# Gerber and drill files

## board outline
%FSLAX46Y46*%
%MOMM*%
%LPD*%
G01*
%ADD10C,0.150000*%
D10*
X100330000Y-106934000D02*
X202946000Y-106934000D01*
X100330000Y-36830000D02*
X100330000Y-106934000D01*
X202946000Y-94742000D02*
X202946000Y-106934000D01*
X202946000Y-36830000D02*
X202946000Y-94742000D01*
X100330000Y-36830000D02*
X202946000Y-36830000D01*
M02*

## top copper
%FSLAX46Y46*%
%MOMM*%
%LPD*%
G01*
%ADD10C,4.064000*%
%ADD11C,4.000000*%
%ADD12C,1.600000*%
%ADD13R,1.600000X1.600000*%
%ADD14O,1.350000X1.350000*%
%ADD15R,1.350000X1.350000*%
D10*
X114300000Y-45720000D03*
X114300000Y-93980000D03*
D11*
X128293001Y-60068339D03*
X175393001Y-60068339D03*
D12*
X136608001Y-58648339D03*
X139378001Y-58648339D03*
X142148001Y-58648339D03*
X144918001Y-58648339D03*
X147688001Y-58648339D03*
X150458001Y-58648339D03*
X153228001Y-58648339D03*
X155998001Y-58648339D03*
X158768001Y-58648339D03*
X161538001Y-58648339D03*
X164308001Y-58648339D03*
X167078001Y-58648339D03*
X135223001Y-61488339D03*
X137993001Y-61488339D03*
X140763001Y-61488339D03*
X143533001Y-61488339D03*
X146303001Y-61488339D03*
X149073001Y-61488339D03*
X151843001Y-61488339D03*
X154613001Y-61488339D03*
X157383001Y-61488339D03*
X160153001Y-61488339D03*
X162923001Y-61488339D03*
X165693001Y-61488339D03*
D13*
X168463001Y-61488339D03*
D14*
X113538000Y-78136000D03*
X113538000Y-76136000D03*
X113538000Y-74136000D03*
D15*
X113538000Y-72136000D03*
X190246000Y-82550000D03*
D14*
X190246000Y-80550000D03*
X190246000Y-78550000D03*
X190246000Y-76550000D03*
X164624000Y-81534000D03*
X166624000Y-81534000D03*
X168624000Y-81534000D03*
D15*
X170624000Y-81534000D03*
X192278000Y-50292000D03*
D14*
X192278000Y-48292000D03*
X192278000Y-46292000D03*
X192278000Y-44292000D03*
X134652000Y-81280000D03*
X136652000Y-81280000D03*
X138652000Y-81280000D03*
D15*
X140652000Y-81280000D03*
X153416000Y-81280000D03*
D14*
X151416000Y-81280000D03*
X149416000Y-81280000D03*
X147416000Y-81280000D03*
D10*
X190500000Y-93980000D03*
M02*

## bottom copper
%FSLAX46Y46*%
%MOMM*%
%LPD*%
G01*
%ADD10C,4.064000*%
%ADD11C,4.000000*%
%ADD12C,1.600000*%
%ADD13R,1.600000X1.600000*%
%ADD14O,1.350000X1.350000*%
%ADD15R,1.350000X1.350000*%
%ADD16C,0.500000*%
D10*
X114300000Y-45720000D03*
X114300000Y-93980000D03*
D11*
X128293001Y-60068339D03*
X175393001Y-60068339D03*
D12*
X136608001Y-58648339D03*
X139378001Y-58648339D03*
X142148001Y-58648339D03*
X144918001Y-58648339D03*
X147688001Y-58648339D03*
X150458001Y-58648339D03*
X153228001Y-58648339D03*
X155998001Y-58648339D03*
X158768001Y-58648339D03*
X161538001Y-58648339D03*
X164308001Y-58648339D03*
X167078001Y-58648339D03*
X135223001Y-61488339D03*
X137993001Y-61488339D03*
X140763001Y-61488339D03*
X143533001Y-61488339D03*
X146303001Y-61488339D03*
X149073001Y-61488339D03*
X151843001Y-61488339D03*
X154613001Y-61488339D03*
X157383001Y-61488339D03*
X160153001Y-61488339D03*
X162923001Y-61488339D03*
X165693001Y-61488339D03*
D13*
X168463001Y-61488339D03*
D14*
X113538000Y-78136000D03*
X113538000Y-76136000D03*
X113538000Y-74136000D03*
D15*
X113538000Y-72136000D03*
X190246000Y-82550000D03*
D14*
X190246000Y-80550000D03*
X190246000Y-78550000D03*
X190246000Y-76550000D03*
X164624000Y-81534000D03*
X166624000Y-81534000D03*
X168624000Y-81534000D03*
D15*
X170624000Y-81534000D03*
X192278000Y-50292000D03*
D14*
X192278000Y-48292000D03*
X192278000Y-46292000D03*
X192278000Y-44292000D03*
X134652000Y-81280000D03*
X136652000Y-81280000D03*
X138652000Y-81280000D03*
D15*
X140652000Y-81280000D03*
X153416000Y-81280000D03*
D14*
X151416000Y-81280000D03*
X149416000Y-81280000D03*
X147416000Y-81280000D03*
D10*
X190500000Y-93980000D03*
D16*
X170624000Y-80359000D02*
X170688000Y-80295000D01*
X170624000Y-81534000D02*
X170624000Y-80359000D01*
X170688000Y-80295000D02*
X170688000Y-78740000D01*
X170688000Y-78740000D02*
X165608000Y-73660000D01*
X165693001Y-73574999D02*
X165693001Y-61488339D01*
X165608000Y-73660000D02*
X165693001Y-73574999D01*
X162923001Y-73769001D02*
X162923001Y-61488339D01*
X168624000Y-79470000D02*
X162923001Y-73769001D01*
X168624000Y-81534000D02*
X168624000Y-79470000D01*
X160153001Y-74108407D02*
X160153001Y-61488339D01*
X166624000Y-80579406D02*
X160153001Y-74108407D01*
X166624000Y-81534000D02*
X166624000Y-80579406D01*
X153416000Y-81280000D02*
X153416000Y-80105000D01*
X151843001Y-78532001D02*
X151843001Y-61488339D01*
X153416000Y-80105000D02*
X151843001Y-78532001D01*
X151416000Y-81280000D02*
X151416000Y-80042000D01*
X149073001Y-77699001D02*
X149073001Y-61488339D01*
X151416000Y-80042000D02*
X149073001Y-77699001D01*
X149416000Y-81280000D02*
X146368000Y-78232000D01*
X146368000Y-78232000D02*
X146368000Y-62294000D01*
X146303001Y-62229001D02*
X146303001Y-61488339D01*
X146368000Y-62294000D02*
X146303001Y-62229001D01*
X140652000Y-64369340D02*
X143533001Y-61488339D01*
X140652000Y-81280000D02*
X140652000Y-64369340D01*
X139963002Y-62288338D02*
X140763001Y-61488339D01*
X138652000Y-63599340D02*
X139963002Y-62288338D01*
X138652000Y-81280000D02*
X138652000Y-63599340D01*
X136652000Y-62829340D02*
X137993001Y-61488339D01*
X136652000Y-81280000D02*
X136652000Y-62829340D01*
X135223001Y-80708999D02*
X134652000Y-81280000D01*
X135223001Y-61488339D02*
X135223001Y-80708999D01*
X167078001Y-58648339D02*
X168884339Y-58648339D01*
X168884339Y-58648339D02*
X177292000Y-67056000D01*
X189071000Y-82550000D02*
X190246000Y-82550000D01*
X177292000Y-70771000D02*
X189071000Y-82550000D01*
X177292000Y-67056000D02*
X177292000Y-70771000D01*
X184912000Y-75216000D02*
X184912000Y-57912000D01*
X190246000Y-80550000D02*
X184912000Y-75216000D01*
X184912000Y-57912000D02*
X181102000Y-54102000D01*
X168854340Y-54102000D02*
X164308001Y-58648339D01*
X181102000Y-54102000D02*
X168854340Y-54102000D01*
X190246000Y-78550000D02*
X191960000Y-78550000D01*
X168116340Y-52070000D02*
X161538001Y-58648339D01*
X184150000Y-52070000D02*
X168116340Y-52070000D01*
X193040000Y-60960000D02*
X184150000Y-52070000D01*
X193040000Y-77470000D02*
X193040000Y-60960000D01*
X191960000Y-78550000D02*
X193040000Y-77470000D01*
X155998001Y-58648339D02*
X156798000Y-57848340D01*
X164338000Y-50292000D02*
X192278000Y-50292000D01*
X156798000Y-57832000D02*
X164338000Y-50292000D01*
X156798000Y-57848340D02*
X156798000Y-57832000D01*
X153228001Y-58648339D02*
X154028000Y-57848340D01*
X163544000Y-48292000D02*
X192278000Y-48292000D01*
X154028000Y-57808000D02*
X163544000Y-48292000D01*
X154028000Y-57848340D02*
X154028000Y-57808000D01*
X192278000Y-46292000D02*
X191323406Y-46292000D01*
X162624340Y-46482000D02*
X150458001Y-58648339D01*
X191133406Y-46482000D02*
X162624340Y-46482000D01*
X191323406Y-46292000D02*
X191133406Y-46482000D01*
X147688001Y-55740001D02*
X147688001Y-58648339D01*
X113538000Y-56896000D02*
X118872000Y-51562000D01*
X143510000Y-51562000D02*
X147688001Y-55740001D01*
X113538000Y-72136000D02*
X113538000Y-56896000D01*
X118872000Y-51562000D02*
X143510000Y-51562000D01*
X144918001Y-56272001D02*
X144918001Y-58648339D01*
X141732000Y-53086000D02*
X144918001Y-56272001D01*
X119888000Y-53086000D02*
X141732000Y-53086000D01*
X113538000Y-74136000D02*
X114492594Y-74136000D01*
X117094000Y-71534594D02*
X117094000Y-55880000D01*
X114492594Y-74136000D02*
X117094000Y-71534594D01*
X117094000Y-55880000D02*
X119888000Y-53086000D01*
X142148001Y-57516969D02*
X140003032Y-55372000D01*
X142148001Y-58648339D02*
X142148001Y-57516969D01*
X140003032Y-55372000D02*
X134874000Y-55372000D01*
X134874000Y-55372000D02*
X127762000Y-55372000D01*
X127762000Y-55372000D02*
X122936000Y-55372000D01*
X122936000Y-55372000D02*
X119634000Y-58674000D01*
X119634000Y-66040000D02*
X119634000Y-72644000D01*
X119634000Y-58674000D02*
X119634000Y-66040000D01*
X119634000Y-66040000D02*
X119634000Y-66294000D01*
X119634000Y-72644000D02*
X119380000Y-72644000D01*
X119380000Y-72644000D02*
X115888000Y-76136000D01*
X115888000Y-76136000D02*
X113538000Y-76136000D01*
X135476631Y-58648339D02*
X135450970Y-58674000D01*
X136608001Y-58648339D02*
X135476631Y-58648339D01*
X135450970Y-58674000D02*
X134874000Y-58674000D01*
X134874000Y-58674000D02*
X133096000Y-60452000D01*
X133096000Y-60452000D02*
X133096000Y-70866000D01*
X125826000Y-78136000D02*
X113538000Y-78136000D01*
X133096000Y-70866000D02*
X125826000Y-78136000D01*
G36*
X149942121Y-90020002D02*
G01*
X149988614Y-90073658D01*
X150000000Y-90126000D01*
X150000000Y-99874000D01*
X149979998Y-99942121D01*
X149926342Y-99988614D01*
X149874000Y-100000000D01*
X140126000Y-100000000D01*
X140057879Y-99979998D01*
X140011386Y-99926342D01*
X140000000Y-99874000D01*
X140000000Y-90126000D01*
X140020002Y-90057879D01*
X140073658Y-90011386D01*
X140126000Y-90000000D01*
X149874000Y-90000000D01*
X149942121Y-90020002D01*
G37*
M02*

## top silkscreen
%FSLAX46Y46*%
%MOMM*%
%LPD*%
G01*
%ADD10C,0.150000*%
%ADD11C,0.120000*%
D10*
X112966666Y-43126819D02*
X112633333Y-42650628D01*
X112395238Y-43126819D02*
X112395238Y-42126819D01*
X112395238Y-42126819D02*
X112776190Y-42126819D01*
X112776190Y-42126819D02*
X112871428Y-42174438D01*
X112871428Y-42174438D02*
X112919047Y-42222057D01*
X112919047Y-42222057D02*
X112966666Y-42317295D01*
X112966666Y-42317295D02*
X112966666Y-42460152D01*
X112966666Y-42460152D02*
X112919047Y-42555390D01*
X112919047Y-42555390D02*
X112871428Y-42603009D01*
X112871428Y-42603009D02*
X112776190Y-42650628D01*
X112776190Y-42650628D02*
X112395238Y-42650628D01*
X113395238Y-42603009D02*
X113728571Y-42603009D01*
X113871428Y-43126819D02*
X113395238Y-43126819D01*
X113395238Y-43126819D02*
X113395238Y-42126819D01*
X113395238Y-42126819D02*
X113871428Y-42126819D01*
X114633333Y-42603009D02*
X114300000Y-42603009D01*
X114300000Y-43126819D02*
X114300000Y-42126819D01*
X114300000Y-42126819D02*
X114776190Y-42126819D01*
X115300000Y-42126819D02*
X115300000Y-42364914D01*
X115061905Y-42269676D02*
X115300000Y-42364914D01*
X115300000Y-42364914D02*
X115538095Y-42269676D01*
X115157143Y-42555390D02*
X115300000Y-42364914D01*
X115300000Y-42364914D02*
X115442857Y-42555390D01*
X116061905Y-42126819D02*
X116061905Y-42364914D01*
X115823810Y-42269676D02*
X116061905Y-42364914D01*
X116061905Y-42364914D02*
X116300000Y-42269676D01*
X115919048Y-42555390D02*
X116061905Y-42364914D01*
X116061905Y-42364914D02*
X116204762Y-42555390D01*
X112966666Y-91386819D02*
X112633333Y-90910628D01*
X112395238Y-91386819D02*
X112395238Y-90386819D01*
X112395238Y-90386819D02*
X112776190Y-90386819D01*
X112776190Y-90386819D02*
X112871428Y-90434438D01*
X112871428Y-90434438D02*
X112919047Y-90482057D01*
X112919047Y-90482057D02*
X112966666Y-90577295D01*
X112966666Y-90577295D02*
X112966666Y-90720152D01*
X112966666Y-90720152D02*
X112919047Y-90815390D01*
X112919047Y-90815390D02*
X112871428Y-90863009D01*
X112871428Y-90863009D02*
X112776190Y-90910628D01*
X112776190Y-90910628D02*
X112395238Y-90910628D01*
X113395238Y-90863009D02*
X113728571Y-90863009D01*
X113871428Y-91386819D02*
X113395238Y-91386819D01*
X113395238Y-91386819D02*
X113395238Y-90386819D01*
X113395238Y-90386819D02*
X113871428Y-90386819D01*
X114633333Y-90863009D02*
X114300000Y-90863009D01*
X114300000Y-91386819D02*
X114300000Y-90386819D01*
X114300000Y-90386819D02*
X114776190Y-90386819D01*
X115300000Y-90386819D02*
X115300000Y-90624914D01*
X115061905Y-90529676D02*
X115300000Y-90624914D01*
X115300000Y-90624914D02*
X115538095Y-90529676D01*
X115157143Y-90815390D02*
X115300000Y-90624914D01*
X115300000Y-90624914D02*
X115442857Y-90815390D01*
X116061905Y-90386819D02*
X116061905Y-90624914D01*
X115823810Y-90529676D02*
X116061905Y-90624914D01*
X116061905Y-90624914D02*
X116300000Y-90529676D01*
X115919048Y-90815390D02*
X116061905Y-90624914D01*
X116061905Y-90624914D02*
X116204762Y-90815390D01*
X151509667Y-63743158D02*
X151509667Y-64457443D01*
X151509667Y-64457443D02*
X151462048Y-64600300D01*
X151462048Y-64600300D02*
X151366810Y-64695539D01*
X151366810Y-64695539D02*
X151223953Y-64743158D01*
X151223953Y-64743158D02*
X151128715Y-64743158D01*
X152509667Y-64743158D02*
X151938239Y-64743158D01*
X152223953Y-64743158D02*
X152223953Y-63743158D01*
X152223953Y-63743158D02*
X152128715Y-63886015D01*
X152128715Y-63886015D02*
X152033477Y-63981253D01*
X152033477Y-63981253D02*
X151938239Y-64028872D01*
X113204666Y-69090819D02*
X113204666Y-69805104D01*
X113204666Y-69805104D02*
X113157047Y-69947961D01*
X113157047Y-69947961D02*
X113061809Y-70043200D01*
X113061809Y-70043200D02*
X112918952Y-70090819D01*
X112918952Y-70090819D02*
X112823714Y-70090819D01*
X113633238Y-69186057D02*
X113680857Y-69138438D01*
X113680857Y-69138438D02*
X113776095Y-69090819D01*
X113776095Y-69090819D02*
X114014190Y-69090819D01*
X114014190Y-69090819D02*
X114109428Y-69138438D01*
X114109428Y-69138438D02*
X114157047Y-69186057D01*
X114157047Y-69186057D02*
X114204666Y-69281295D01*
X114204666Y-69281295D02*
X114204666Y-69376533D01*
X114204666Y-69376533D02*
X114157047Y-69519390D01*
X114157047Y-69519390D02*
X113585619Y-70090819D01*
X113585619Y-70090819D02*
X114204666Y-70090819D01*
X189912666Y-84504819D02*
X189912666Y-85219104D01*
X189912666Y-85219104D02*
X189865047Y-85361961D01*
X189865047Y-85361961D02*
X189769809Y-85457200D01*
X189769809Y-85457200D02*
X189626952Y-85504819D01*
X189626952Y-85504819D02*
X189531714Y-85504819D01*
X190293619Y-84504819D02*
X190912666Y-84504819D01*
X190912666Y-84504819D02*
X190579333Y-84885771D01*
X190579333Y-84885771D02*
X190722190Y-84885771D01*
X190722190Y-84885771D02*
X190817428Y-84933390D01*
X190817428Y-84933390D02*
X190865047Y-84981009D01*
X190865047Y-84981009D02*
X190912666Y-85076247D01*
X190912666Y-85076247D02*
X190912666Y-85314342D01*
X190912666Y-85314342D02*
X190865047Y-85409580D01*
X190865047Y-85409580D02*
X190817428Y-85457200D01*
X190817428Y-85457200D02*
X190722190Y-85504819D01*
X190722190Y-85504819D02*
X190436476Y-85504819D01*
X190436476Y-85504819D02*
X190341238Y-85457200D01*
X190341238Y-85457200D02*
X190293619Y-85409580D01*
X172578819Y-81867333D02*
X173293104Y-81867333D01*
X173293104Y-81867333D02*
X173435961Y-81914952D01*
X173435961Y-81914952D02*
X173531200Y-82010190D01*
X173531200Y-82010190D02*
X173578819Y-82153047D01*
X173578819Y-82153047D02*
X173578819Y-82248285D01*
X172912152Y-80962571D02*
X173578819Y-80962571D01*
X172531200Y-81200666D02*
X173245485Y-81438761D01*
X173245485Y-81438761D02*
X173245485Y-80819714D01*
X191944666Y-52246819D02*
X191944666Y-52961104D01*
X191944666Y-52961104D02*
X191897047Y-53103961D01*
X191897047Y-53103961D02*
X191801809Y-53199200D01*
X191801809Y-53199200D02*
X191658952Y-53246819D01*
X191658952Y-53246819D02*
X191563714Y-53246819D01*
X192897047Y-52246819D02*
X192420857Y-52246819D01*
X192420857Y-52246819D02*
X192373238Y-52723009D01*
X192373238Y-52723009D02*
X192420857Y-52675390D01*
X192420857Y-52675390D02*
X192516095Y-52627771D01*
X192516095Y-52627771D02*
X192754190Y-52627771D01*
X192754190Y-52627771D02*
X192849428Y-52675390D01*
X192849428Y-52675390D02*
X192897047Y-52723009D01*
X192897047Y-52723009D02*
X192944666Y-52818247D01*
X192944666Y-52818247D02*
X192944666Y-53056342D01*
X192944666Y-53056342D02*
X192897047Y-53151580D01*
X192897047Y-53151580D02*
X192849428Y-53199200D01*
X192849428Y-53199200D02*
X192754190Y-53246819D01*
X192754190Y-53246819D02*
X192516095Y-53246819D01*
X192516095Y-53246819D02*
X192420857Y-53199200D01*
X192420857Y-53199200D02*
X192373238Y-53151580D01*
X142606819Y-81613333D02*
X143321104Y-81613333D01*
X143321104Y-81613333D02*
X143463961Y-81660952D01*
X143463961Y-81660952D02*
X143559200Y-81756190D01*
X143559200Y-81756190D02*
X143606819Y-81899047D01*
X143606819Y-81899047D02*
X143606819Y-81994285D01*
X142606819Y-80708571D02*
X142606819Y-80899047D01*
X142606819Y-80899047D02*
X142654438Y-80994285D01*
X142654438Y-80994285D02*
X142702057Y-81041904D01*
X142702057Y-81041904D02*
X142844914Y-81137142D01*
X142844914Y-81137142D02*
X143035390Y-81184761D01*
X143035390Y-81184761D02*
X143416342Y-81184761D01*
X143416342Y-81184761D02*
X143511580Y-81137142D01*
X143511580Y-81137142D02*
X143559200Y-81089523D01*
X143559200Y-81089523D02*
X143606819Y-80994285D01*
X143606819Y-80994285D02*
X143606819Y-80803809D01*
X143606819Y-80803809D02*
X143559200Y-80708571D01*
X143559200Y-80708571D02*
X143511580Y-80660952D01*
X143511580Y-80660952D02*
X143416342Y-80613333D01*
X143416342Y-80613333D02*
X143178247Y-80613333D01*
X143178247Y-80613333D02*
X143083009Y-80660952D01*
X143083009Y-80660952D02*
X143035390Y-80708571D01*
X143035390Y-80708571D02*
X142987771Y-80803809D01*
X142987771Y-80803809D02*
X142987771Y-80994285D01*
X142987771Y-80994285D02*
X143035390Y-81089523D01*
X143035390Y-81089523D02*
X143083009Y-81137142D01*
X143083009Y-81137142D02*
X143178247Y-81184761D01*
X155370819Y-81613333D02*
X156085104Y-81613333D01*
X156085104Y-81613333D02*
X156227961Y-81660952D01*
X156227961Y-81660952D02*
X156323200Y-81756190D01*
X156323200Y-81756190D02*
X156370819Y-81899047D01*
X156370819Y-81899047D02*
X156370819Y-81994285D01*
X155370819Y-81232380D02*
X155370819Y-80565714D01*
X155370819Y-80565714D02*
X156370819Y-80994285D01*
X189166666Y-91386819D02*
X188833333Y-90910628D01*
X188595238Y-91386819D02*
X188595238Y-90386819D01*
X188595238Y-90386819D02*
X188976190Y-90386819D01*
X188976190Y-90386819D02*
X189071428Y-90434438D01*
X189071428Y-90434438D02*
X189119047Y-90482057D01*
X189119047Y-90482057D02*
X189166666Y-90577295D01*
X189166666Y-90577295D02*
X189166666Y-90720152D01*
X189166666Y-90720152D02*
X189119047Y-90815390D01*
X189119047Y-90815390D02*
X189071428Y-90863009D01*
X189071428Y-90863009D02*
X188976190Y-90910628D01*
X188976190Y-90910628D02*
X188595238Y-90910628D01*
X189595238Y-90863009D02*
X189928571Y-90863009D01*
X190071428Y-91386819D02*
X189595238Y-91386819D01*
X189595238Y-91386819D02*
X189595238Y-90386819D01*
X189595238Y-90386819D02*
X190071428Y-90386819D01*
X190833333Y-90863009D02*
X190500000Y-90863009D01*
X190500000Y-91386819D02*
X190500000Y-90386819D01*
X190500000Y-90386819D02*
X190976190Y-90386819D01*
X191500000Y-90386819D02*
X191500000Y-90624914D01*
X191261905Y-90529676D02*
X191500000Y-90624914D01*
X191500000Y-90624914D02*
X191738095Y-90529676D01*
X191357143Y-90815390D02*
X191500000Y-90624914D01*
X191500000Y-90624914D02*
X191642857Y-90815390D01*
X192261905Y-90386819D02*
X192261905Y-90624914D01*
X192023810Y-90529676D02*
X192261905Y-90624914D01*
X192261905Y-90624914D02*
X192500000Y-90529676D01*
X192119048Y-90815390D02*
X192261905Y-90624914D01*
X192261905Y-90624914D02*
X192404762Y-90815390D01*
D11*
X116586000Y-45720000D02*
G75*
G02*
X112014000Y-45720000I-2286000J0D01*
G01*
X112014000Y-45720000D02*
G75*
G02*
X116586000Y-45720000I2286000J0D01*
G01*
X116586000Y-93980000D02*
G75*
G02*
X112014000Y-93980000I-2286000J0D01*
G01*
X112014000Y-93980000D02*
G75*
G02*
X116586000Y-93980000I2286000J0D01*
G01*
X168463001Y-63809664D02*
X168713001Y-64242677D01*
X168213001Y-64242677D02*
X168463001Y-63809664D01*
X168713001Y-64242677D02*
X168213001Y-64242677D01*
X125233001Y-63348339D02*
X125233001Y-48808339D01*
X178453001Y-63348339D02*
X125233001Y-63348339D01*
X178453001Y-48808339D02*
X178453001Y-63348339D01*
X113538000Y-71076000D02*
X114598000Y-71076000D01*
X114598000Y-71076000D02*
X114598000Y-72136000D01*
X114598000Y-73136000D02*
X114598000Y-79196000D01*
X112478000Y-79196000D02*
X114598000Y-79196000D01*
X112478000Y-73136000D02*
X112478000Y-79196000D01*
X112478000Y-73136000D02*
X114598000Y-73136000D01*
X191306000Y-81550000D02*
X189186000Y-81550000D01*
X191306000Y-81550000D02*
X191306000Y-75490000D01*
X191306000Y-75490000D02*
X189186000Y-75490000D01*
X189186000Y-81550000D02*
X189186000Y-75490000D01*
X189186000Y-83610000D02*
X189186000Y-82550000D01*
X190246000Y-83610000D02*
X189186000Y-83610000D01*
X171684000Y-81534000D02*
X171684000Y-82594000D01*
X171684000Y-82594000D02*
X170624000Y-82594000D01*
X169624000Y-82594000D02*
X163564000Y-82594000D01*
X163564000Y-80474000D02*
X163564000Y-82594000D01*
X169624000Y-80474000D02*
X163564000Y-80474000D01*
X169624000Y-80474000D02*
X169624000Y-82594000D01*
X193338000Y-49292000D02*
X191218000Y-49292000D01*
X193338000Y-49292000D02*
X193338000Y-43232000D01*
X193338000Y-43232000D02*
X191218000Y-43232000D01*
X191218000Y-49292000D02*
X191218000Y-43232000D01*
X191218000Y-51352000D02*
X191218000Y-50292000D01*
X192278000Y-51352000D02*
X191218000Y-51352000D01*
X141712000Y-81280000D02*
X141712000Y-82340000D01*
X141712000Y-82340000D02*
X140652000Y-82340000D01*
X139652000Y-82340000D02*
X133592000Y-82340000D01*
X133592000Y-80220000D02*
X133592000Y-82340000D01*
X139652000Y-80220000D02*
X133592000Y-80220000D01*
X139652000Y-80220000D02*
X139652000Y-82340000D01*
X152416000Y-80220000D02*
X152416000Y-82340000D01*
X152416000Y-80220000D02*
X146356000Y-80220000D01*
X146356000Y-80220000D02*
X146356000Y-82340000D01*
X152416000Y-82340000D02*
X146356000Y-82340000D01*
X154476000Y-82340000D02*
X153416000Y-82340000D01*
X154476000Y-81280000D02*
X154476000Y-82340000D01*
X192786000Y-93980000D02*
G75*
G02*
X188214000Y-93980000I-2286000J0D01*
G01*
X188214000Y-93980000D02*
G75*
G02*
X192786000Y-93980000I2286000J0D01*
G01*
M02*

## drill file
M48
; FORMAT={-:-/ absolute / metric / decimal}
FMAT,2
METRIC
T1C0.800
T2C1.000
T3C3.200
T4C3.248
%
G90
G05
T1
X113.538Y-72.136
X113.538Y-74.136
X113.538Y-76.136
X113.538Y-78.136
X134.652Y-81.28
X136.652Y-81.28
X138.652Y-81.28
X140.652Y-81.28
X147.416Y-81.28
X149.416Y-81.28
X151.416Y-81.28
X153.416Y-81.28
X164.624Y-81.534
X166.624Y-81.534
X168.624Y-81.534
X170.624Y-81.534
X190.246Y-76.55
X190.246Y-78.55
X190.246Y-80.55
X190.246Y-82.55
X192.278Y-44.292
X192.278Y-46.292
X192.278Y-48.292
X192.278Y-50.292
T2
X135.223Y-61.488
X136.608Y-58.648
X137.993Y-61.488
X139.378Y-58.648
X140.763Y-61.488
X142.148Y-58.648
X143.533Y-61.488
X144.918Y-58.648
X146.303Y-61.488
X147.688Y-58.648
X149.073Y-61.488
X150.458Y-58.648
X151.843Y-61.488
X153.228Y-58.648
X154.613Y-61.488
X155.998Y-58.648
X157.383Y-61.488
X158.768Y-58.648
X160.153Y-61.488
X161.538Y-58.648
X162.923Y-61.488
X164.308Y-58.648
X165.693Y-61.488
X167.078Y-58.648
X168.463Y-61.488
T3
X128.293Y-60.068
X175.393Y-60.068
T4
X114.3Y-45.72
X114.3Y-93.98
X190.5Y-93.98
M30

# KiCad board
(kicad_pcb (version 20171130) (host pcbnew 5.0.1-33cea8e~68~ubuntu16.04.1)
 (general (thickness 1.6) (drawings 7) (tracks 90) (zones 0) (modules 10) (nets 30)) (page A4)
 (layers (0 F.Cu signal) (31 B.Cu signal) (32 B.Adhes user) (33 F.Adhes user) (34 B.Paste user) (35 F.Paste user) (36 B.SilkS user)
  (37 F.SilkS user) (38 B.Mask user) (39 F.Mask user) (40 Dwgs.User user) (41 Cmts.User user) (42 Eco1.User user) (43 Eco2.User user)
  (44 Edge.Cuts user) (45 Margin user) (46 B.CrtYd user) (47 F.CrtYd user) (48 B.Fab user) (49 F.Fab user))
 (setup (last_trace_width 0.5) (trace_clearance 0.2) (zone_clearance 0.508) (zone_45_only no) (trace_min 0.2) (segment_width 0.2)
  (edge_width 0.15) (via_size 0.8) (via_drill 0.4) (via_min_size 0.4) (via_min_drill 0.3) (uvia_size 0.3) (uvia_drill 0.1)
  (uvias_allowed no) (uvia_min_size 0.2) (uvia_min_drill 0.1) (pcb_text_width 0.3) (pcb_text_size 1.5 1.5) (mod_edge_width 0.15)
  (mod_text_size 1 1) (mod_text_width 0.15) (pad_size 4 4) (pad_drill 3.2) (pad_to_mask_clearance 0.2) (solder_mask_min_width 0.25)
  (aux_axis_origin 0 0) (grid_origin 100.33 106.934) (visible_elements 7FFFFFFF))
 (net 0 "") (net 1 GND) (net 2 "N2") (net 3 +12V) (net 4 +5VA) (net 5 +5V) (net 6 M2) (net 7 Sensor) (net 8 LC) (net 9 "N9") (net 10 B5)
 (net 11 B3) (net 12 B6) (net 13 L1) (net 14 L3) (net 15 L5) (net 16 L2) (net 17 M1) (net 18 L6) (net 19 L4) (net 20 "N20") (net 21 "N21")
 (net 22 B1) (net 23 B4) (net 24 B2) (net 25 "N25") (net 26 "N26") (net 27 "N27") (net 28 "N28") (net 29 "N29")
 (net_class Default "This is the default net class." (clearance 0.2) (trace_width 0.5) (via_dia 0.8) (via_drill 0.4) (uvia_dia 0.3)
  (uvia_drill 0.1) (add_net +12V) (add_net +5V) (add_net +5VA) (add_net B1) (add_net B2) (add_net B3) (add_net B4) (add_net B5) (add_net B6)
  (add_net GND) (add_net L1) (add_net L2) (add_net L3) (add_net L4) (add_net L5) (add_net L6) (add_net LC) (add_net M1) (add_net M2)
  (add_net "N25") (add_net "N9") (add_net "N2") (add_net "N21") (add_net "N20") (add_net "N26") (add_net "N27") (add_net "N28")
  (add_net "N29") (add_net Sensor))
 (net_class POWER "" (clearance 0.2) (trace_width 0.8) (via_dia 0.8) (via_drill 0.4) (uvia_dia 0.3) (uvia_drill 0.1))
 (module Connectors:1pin (layer F.Cu) (at 114.3 45.72)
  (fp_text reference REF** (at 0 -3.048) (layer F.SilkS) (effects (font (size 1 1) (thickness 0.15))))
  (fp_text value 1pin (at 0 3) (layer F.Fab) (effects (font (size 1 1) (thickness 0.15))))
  (fp_circle (center 0 0) (end 0 -2.286) (layer F.SilkS) (width 0.12))
  (pad 1 thru_hole circle (at 0 0) (size 4.064 4.064) (drill 3.248) (layers *.Cu *.Mask)))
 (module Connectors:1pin (layer F.Cu) (at 114.3 93.98)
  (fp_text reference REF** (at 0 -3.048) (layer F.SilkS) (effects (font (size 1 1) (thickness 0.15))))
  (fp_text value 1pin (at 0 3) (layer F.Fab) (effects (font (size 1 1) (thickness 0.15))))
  (fp_circle (center 0 0) (end 0 -2.286) (layer F.SilkS) (width 0.12))
  (pad 1 thru_hole circle (at 0 0) (size 4.064 4.064) (drill 3.248) (layers *.Cu *.Mask)))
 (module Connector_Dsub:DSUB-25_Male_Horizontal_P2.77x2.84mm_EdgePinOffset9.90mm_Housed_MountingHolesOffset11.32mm (layer F.Cu)
  (at 168.463001 61.488339 180)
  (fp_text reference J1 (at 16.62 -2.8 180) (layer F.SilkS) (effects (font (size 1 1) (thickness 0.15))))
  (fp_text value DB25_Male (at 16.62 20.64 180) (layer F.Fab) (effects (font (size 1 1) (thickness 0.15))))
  (fp_line (start 0 -2.321325) (end -0.25 -2.754338) (layer F.SilkS) (width 0.12))
  (fp_line (start 0.25 -2.754338) (end 0 -2.321325) (layer F.SilkS) (width 0.12))
  (fp_line (start -0.25 -2.754338) (end 0.25 -2.754338) (layer F.SilkS) (width 0.12))
  (fp_line (start 43.23 -1.86) (end 43.23 12.68) (layer F.SilkS) (width 0.12))
  (fp_line (start -9.99 -1.86) (end 43.23 -1.86) (layer F.SilkS) (width 0.12))
  (fp_line (start -9.99 12.68) (end -9.99 -1.86) (layer F.SilkS) (width 0.12))
  (pad 0 thru_hole circle (at 40.17 1.42 180) (size 4 4) (drill 3.2) (layers *.Cu *.Mask))
  (pad 0 thru_hole circle (at -6.93 1.42 180) (size 4 4) (drill 3.2) (layers *.Cu *.Mask))
  (pad 25 thru_hole circle (at 31.855 2.84 180) (size 1.6 1.6) (drill 1) (layers *.Cu *.Mask) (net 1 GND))
  (pad 24 thru_hole circle (at 29.085 2.84 180) (size 1.6 1.6) (drill 1) (layers *.Cu *.Mask) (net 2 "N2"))
  (pad 23 thru_hole circle (at 26.315 2.84 180) (size 1.6 1.6) (drill 1) (layers *.Cu *.Mask) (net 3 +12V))
  (pad 22 thru_hole circle (at 23.545 2.84 180) (size 1.6 1.6) (drill 1) (layers *.Cu *.Mask) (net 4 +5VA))
  (pad 21 thru_hole circle (at 20.775 2.84 180) (size 1.6 1.6) (drill 1) (layers *.Cu *.Mask) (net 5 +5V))
  (pad 20 thru_hole circle (at 18.005 2.84 180) (size 1.6 1.6) (drill 1) (layers *.Cu *.Mask) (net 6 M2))
  (pad 19 thru_hole circle (at 15.235 2.84 180) (size 1.6 1.6) (drill 1) (layers *.Cu *.Mask) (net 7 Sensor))
  (pad 18 thru_hole circle (at 12.465 2.84 180) (size 1.6 1.6) (drill 1) (layers *.Cu *.Mask) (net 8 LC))
  (pad 17 thru_hole circle (at 9.695 2.84 180) (size 1.6 1.6) (drill 1) (layers *.Cu *.Mask) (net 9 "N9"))
  (pad 16 thru_hole circle (at 6.925 2.84 180) (size 1.6 1.6) (drill 1) (layers *.Cu *.Mask) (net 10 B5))
  (pad 15 thru_hole circle (at 4.155 2.84 180) (size 1.6 1.6) (drill 1) (layers *.Cu *.Mask) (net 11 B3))
  (pad 14 thru_hole circle (at 1.385 2.84 180) (size 1.6 1.6) (drill 1) (layers *.Cu *.Mask) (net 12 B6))
  (pad 13 thru_hole circle (at 33.24 0 180) (size 1.6 1.6) (drill 1) (layers *.Cu *.Mask) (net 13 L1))
  (pad 12 thru_hole circle (at 30.47 0 180) (size 1.6 1.6) (drill 1) (layers *.Cu *.Mask) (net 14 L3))
  (pad 11 thru_hole circle (at 27.7 0 180) (size 1.6 1.6) (drill 1) (layers *.Cu *.Mask) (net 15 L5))
  (pad 10 thru_hole circle (at 24.93 0 180) (size 1.6 1.6) (drill 1) (layers *.Cu *.Mask) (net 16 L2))
  (pad 9 thru_hole circle (at 22.16 0 180) (size 1.6 1.6) (drill 1) (layers *.Cu *.Mask) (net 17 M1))
  (pad 8 thru_hole circle (at 19.39 0 180) (size 1.6 1.6) (drill 1) (layers *.Cu *.Mask) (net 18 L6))
  (pad 7 thru_hole circle (at 16.62 0 180) (size 1.6 1.6) (drill 1) (layers *.Cu *.Mask) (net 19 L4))
  (pad 6 thru_hole circle (at 13.85 0 180) (size 1.6 1.6) (drill 1) (layers *.Cu *.Mask) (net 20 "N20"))
  (pad 5 thru_hole circle (at 11.08 0 180) (size 1.6 1.6) (drill 1) (layers *.Cu *.Mask) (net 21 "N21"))
  (pad 4 thru_hole circle (at 8.31 0 180) (size 1.6 1.6) (drill 1) (layers *.Cu *.Mask) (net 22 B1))
  (pad 3 thru_hole circle (at 5.54 0 180) (size 1.6 1.6) (drill 1) (layers *.Cu *.Mask) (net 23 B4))
  (pad 2 thru_hole circle (at 2.77 0 180) (size 1.6 1.6) (drill 1) (layers *.Cu *.Mask) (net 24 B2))
  (pad 1 thru_hole rect (at 0 0 180) (size 1.6 1.6) (drill 1) (layers *.Cu *.Mask) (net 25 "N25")))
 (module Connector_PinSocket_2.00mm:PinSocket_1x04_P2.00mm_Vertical (layer F.Cu) (at 113.538 72.136)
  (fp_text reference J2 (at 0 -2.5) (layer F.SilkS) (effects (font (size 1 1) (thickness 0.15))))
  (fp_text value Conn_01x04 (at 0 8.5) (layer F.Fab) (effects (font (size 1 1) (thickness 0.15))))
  (fp_line (start 0 -1.06) (end 1.06 -1.06) (layer F.SilkS) (width 0.12))
  (fp_line (start 1.06 -1.06) (end 1.06 0) (layer F.SilkS) (width 0.12))
  (fp_line (start 1.06 1) (end 1.06 7.06) (layer F.SilkS) (width 0.12))
  (fp_line (start -1.06 7.06) (end 1.06 7.06) (layer F.SilkS) (width 0.12))
  (fp_line (start -1.06 1) (end -1.06 7.06) (layer F.SilkS) (width 0.12))
  (fp_line (start -1.06 1) (end 1.06 1) (layer F.SilkS) (width 0.12))
  (pad 4 thru_hole oval (at 0 6) (size 1.35 1.35) (drill 0.8) (layers *.Cu *.Mask) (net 1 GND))
  (pad 3 thru_hole oval (at 0 4) (size 1.35 1.35) (drill 0.8) (layers *.Cu *.Mask) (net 3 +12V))
  (pad 2 thru_hole oval (at 0 2) (size 1.35 1.35) (drill 0.8) (layers *.Cu *.Mask) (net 4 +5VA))
  (pad 1 thru_hole rect (at 0 0) (size 1.35 1.35) (drill 0.8) (layers *.Cu *.Mask) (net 5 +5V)))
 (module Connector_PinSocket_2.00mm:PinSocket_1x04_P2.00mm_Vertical (layer F.Cu) (at 190.246 82.55 180)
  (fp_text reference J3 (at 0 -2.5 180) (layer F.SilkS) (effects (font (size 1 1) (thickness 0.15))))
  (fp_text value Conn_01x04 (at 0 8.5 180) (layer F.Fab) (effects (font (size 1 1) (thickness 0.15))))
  (fp_line (start -1.06 1) (end 1.06 1) (layer F.SilkS) (width 0.12))
  (fp_line (start -1.06 1) (end -1.06 7.06) (layer F.SilkS) (width 0.12))
  (fp_line (start -1.06 7.06) (end 1.06 7.06) (layer F.SilkS) (width 0.12))
  (fp_line (start 1.06 1) (end 1.06 7.06) (layer F.SilkS) (width 0.12))
  (fp_line (start 1.06 -1.06) (end 1.06 0) (layer F.SilkS) (width 0.12))
  (fp_line (start 0 -1.06) (end 1.06 -1.06) (layer F.SilkS) (width 0.12))
  (pad 1 thru_hole rect (at 0 0 180) (size 1.35 1.35) (drill 0.8) (layers *.Cu *.Mask) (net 12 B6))
  (pad 2 thru_hole oval (at 0 2 180) (size 1.35 1.35) (drill 0.8) (layers *.Cu *.Mask) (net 11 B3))
  (pad 3 thru_hole oval (at 0 4 180) (size 1.35 1.35) (drill 0.8) (layers *.Cu *.Mask) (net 10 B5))
  (pad 4 thru_hole oval (at 0 6 180) (size 1.35 1.35) (drill 0.8) (layers *.Cu *.Mask) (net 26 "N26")))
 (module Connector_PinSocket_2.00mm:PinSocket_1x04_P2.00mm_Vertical (layer F.Cu) (at 170.624 81.534 270)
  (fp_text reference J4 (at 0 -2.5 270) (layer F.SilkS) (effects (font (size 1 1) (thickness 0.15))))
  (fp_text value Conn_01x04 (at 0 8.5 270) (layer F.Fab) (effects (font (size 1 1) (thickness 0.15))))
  (fp_line (start 0 -1.06) (end 1.06 -1.06) (layer F.SilkS) (width 0.12))
  (fp_line (start 1.06 -1.06) (end 1.06 0) (layer F.SilkS) (width 0.12))
  (fp_line (start 1.06 1) (end 1.06 7.06) (layer F.SilkS) (width 0.12))
  (fp_line (start -1.06 7.06) (end 1.06 7.06) (layer F.SilkS) (width 0.12))
  (fp_line (start -1.06 1) (end -1.06 7.06) (layer F.SilkS) (width 0.12))
  (fp_line (start -1.06 1) (end 1.06 1) (layer F.SilkS) (width 0.12))
  (pad 4 thru_hole oval (at 0 6 270) (size 1.35 1.35) (drill 0.8) (layers *.Cu *.Mask) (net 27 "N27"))
  (pad 3 thru_hole oval (at 0 4 270) (size 1.35 1.35) (drill 0.8) (layers *.Cu *.Mask) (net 22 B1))
  (pad 2 thru_hole oval (at 0 2 270) (size 1.35 1.35) (drill 0.8) (layers *.Cu *.Mask) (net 23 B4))
  (pad 1 thru_hole rect (at 0 0 270) (size 1.35 1.35) (drill 0.8) (layers *.Cu *.Mask) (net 24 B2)))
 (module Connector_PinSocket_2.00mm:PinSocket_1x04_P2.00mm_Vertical (layer F.Cu) (at 192.278 50.292 180)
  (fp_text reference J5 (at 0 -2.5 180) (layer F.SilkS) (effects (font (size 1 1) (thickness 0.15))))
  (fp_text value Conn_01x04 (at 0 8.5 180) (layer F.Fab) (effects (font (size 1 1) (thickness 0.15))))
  (fp_line (start -1.06 1) (end 1.06 1) (layer F.SilkS) (width 0.12))
  (fp_line (start -1.06 1) (end -1.06 7.06) (layer F.SilkS) (width 0.12))
  (fp_line (start -1.06 7.06) (end 1.06 7.06) (layer F.SilkS) (width 0.12))
  (fp_line (start 1.06 1) (end 1.06 7.06) (layer F.SilkS) (width 0.12))
  (fp_line (start 1.06 -1.06) (end 1.06 0) (layer F.SilkS) (width 0.12))
  (fp_line (start 0 -1.06) (end 1.06 -1.06) (layer F.SilkS) (width 0.12))
  (pad 1 thru_hole rect (at 0 0 180) (size 1.35 1.35) (drill 0.8) (layers *.Cu *.Mask) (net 8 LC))
  (pad 2 thru_hole oval (at 0 2 180) (size 1.35 1.35) (drill 0.8) (layers *.Cu *.Mask) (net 7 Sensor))
  (pad 3 thru_hole oval (at 0 4 180) (size 1.35 1.35) (drill 0.8) (layers *.Cu *.Mask) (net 6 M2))
  (pad 4 thru_hole oval (at 0 6 180) (size 1.35 1.35) (drill 0.8) (layers *.Cu *.Mask) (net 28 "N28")))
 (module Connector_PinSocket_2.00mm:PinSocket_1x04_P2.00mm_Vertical (layer F.Cu) (at 140.652 81.28 270)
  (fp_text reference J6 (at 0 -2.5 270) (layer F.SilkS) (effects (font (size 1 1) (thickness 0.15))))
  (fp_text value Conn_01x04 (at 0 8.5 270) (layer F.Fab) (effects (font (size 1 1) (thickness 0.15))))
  (fp_line (start 0 -1.06) (end 1.06 -1.06) (layer F.SilkS) (width 0.12))
  (fp_line (start 1.06 -1.06) (end 1.06 0) (layer F.SilkS) (width 0.12))
  (fp_line (start 1.06 1) (end 1.06 7.06) (layer F.SilkS) (width 0.12))
  (fp_line (start -1.06 7.06) (end 1.06 7.06) (layer F.SilkS) (width 0.12))
  (fp_line (start -1.06 1) (end -1.06 7.06) (layer F.SilkS) (width 0.12))
  (fp_line (start -1.06 1) (end 1.06 1) (layer F.SilkS) (width 0.12))
  (pad 4 thru_hole oval (at 0 6 270) (size 1.35 1.35) (drill 0.8) (layers *.Cu *.Mask) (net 13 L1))
  (pad 3 thru_hole oval (at 0 4 270) (size 1.35 1.35) (drill 0.8) (layers *.Cu *.Mask) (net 14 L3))
  (pad 2 thru_hole oval (at 0 2 270) (size 1.35 1.35) (drill 0.8) (layers *.Cu *.Mask) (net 15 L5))
  (pad 1 thru_hole rect (at 0 0 270) (size 1.35 1.35) (drill 0.8) (layers *.Cu *.Mask) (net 16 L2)))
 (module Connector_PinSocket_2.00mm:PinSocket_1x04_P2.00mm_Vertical (layer F.Cu) (at 153.416 81.28 270)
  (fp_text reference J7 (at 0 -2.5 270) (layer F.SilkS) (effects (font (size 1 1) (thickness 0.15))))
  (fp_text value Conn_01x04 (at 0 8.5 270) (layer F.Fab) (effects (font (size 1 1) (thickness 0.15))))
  (fp_line (start -1.06 1) (end 1.06 1) (layer F.SilkS) (width 0.12))
  (fp_line (start -1.06 1) (end -1.06 7.06) (layer F.SilkS) (width 0.12))
  (fp_line (start -1.06 7.06) (end 1.06 7.06) (layer F.SilkS) (width 0.12))
  (fp_line (start 1.06 1) (end 1.06 7.06) (layer F.SilkS) (width 0.12))
  (fp_line (start 1.06 -1.06) (end 1.06 0) (layer F.SilkS) (width 0.12))
  (fp_line (start 0 -1.06) (end 1.06 -1.06) (layer F.SilkS) (width 0.12))
  (pad 1 thru_hole rect (at 0 0 270) (size 1.35 1.35) (drill 0.8) (layers *.Cu *.Mask) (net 19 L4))
  (pad 2 thru_hole oval (at 0 2 270) (size 1.35 1.35) (drill 0.8) (layers *.Cu *.Mask) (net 18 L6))
  (pad 3 thru_hole oval (at 0 4 270) (size 1.35 1.35) (drill 0.8) (layers *.Cu *.Mask) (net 17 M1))
  (pad 4 thru_hole oval (at 0 6 270) (size 1.35 1.35) (drill 0.8) (layers *.Cu *.Mask) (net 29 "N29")))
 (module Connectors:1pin (layer F.Cu) (at 190.5 93.98)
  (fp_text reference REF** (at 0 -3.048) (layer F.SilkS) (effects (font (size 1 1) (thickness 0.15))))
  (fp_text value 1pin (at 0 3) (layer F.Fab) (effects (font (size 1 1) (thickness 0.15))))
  (fp_circle (center 0 0) (end 0 -2.286) (layer F.SilkS) (width 0.12))
  (pad 1 thru_hole circle (at 0 0) (size 4.064 4.064) (drill 3.248) (layers *.Cu *.Mask)))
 (gr_line (start 100.33 106.934) (end 202.946 106.934) (layer Edge.Cuts) (width 0.15))
 (gr_line (start 100.33 36.83) (end 100.33 106.934) (layer Edge.Cuts) (width 0.15))
 (gr_line (start 202.946 94.742) (end 202.946 106.934) (layer Edge.Cuts) (width 0.15))
 (gr_line (start 202.946 36.83) (end 202.946 94.742) (layer Edge.Cuts) (width 0.15))
 (gr_line (start 100.33 36.83) (end 202.946 36.83) (layer Edge.Cuts) (width 0.15))
 (segment (start 170.624 80.359) (end 170.688 80.295) (width 0.5) (layer B.Cu) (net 24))
 (segment (start 170.624 81.534) (end 170.624 80.359) (width 0.5) (layer B.Cu) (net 24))
 (segment (start 170.688 80.295) (end 170.688 78.74) (width 0.5) (layer B.Cu) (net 24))
 (segment (start 170.688 78.74) (end 165.608 73.66) (width 0.5) (layer B.Cu) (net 24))
 (segment (start 165.693001 73.574999) (end 165.693001 61.488339) (width 0.5) (layer B.Cu) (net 24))
 (segment (start 165.608 73.66) (end 165.693001 73.574999) (width 0.5) (layer B.Cu) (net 24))
 (segment (start 162.923001 73.769001) (end 162.923001 61.488339) (width 0.5) (layer B.Cu) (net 23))
 (segment (start 168.624 79.47) (end 162.923001 73.769001) (width 0.5) (layer B.Cu) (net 23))
 (segment (start 168.624 81.534) (end 168.624 79.47) (width 0.5) (layer B.Cu) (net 23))
 (segment (start 160.153001 74.108407) (end 160.153001 61.488339) (width 0.5) (layer B.Cu) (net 22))
 (segment (start 166.624 80.579406) (end 160.153001 74.108407) (width 0.5) (layer B.Cu) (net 22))
 (segment (start 166.624 81.534) (end 166.624 80.579406) (width 0.5) (layer B.Cu) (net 22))
 (segment (start 153.416 81.28) (end 153.416 80.105) (width 0.5) (layer B.Cu) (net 19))
 (segment (start 151.843001 78.532001) (end 151.843001 61.488339) (width 0.5) (layer B.Cu) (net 19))
 (segment (start 153.416 80.105) (end 151.843001 78.532001) (width 0.5) (layer B.Cu) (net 19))
 (segment (start 151.416 81.28) (end 151.416 80.042) (width 0.5) (layer B.Cu) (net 18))
 (segment (start 149.073001 77.699001) (end 149.073001 61.488339) (width 0.5) (layer B.Cu) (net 18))
 (segment (start 151.416 80.042) (end 149.073001 77.699001) (width 0.5) (layer B.Cu) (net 18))
 (segment (start 149.416 81.28) (end 146.368 78.232) (width 0.5) (layer B.Cu) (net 17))
 (segment (start 146.368 78.232) (end 146.368 62.294) (width 0.5) (layer B.Cu) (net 17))
 (segment (start 146.303001 62.229001) (end 146.303001 61.488339) (width 0.5) (layer B.Cu) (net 17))
 (segment (start 146.368 62.294) (end 146.303001 62.229001) (width 0.5) (layer B.Cu) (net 17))
 (segment (start 140.652 64.36934) (end 143.533001 61.488339) (width 0.5) (layer B.Cu) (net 16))
 (segment (start 140.652 81.28) (end 140.652 64.36934) (width 0.5) (layer B.Cu) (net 16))
 (segment (start 139.963002 62.288338) (end 140.763001 61.488339) (width 0.5) (layer B.Cu) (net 15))
 (segment (start 138.652 63.59934) (end 139.963002 62.288338) (width 0.5) (layer B.Cu) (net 15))
 (segment (start 138.652 81.28) (end 138.652 63.59934) (width 0.5) (layer B.Cu) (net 15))
 (segment (start 136.652 62.82934) (end 137.993001 61.488339) (width 0.5) (layer B.Cu) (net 14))
 (segment (start 136.652 81.28) (end 136.652 62.82934) (width 0.5) (layer B.Cu) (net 14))
 (segment (start 135.223001 80.708999) (end 134.652 81.28) (width 0.5) (layer B.Cu) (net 13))
 (segment (start 135.223001 61.488339) (end 135.223001 80.708999) (width 0.5) (layer B.Cu) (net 13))
 (segment (start 167.078001 58.648339) (end 168.884339 58.648339) (width 0.5) (layer B.Cu) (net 12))
 (segment (start 168.884339 58.648339) (end 177.292 67.056) (width 0.5) (layer B.Cu) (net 12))
 (segment (start 189.071 82.55) (end 190.246 82.55) (width 0.5) (layer B.Cu) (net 12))
 (segment (start 177.292 70.771) (end 189.071 82.55) (width 0.5) (layer B.Cu) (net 12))
 (segment (start 177.292 67.056) (end 177.292 70.771) (width 0.5) (layer B.Cu) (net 12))
 (segment (start 184.912 75.216) (end 184.912 57.912) (width 0.5) (layer B.Cu) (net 11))
 (segment (start 190.246 80.55) (end 184.912 75.216) (width 0.5) (layer B.Cu) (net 11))
 (segment (start 184.912 57.912) (end 181.102 54.102) (width 0.5) (layer B.Cu) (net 11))
 (segment (start 168.85434 54.102) (end 164.308001 58.648339) (width 0.5) (layer B.Cu) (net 11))
 (segment (start 181.102 54.102) (end 168.85434 54.102) (width 0.5) (layer B.Cu) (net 11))
 (segment (start 190.246 78.55) (end 191.96 78.55) (width 0.5) (layer B.Cu) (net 10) (status 400000))
 (segment (start 168.11634 52.07) (end 161.538001 58.648339) (width 0.5) (layer B.Cu) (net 10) (status 800000))
 (segment (start 184.15 52.07) (end 168.11634 52.07) (width 0.5) (layer B.Cu) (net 10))
 (segment (start 193.04 60.96) (end 184.15 52.07) (width 0.5) (layer B.Cu) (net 10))
 (segment (start 193.04 77.47) (end 193.04 60.96) (width 0.5) (layer B.Cu) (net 10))
 (segment (start 191.96 78.55) (end 193.04 77.47) (width 0.5) (layer B.Cu) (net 10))
 (segment (start 155.998001 58.648339) (end 156.798 57.84834) (width 0.5) (layer B.Cu) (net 8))
 (segment (start 164.338 50.292) (end 192.278 50.292) (width 0.5) (layer B.Cu) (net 8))
 (segment (start 156.798 57.832) (end 164.338 50.292) (width 0.5) (layer B.Cu) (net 8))
 (segment (start 156.798 57.84834) (end 156.798 57.832) (width 0.5) (layer B.Cu) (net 8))
 (segment (start 153.228001 58.648339) (end 154.028 57.84834) (width 0.5) (layer B.Cu) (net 7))
 (segment (start 163.544 48.292) (end 192.278 48.292) (width 0.5) (layer B.Cu) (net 7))
 (segment (start 154.028 57.808) (end 163.544 48.292) (width 0.5) (layer B.Cu) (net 7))
 (segment (start 154.028 57.84834) (end 154.028 57.808) (width 0.5) (layer B.Cu) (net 7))
 (segment (start 192.278 46.292) (end 191.323406 46.292) (width 0.5) (layer B.Cu) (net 6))
 (segment (start 162.62434 46.482) (end 150.458001 58.648339) (width 0.5) (layer B.Cu) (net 6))
 (segment (start 191.133406 46.482) (end 162.62434 46.482) (width 0.5) (layer B.Cu) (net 6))
 (segment (start 191.323406 46.292) (end 191.133406 46.482) (width 0.5) (layer B.Cu) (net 6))
 (segment (start 147.688001 55.740001) (end 147.688001 58.648339) (width 0.5) (layer B.Cu) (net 5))
 (segment (start 113.538 56.896) (end 118.872 51.562) (width 0.5) (layer B.Cu) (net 5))
 (segment (start 143.51 51.562) (end 147.688001 55.740001) (width 0.5) (layer B.Cu) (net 5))
 (segment (start 113.538 72.136) (end 113.538 56.896) (width 0.5) (layer B.Cu) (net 5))
 (segment (start 118.872 51.562) (end 143.51 51.562) (width 0.5) (layer B.Cu) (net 5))
 (segment (start 144.918001 56.272001) (end 144.918001 58.648339) (width 0.5) (layer B.Cu) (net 4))
 (segment (start 141.732 53.086) (end 144.918001 56.272001) (width 0.5) (layer B.Cu) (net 4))
 (segment (start 119.888 53.086) (end 141.732 53.086) (width 0.5) (layer B.Cu) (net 4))
 (segment (start 113.538 74.136) (end 114.492594 74.136) (width 0.5) (layer B.Cu) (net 4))
 (segment (start 117.094 71.534594) (end 117.094 55.88) (width 0.5) (layer B.Cu) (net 4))
 (segment (start 114.492594 74.136) (end 117.094 71.534594) (width 0.5) (layer B.Cu) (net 4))
 (segment (start 117.094 55.88) (end 119.888 53.086) (width 0.5) (layer B.Cu) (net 4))
 (segment (start 142.148001 57.516969) (end 140.003032 55.372) (width 0.5) (layer B.Cu) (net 3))
 (segment (start 142.148001 58.648339) (end 142.148001 57.516969) (width 0.5) (layer B.Cu) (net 3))
 (segment (start 140.003032 55.372) (end 134.874 55.372) (width 0.5) (layer B.Cu) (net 3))
 (segment (start 134.874 55.372) (end 127.762 55.372) (width 0.5) (layer B.Cu) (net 3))
 (segment (start 127.762 55.372) (end 122.936 55.372) (width 0.5) (layer B.Cu) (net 3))
 (segment (start 122.936 55.372) (end 119.634 58.674) (width 0.5) (layer B.Cu) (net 3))
 (segment (start 119.634 66.04) (end 119.634 72.644) (width 0.5) (layer B.Cu) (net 3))
 (segment (start 119.634 58.674) (end 119.634 66.04) (width 0.5) (layer B.Cu) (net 3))
 (segment (start 119.634 66.04) (end 119.634 66.294) (width 0.5) (layer B.Cu) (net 3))
 (segment (start 119.634 72.644) (end 119.38 72.644) (width 0.5) (layer B.Cu) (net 3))
 (segment (start 119.38 72.644) (end 115.888 76.136) (width 0.5) (layer B.Cu) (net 3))
 (segment (start 115.888 76.136) (end 113.538 76.136) (width 0.5) (layer B.Cu) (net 3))
 (segment (start 135.476631 58.648339) (end 135.45097 58.674) (width 0.5) (layer B.Cu) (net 1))
 (segment (start 136.608001 58.648339) (end 135.476631 58.648339) (width 0.5) (layer B.Cu) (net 1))
 (segment (start 135.45097 58.674) (end 134.874 58.674) (width 0.5) (layer B.Cu) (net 1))
 (segment (start 134.874 58.674) (end 133.096 60.452) (width 0.5) (layer B.Cu) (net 1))
 (segment (start 133.096 60.452) (end 133.096 70.866) (width 0.5) (layer B.Cu) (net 1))
 (segment (start 125.826 78.136) (end 113.538 78.136) (width 0.5) (layer B.Cu) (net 1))
 (segment (start 133.096 70.866) (end 125.826 78.136) (width 0.5) (layer B.Cu) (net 1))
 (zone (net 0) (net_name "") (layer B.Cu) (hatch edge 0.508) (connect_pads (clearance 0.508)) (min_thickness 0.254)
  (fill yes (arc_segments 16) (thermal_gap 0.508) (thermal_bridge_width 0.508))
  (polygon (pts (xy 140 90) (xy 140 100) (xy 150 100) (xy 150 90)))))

